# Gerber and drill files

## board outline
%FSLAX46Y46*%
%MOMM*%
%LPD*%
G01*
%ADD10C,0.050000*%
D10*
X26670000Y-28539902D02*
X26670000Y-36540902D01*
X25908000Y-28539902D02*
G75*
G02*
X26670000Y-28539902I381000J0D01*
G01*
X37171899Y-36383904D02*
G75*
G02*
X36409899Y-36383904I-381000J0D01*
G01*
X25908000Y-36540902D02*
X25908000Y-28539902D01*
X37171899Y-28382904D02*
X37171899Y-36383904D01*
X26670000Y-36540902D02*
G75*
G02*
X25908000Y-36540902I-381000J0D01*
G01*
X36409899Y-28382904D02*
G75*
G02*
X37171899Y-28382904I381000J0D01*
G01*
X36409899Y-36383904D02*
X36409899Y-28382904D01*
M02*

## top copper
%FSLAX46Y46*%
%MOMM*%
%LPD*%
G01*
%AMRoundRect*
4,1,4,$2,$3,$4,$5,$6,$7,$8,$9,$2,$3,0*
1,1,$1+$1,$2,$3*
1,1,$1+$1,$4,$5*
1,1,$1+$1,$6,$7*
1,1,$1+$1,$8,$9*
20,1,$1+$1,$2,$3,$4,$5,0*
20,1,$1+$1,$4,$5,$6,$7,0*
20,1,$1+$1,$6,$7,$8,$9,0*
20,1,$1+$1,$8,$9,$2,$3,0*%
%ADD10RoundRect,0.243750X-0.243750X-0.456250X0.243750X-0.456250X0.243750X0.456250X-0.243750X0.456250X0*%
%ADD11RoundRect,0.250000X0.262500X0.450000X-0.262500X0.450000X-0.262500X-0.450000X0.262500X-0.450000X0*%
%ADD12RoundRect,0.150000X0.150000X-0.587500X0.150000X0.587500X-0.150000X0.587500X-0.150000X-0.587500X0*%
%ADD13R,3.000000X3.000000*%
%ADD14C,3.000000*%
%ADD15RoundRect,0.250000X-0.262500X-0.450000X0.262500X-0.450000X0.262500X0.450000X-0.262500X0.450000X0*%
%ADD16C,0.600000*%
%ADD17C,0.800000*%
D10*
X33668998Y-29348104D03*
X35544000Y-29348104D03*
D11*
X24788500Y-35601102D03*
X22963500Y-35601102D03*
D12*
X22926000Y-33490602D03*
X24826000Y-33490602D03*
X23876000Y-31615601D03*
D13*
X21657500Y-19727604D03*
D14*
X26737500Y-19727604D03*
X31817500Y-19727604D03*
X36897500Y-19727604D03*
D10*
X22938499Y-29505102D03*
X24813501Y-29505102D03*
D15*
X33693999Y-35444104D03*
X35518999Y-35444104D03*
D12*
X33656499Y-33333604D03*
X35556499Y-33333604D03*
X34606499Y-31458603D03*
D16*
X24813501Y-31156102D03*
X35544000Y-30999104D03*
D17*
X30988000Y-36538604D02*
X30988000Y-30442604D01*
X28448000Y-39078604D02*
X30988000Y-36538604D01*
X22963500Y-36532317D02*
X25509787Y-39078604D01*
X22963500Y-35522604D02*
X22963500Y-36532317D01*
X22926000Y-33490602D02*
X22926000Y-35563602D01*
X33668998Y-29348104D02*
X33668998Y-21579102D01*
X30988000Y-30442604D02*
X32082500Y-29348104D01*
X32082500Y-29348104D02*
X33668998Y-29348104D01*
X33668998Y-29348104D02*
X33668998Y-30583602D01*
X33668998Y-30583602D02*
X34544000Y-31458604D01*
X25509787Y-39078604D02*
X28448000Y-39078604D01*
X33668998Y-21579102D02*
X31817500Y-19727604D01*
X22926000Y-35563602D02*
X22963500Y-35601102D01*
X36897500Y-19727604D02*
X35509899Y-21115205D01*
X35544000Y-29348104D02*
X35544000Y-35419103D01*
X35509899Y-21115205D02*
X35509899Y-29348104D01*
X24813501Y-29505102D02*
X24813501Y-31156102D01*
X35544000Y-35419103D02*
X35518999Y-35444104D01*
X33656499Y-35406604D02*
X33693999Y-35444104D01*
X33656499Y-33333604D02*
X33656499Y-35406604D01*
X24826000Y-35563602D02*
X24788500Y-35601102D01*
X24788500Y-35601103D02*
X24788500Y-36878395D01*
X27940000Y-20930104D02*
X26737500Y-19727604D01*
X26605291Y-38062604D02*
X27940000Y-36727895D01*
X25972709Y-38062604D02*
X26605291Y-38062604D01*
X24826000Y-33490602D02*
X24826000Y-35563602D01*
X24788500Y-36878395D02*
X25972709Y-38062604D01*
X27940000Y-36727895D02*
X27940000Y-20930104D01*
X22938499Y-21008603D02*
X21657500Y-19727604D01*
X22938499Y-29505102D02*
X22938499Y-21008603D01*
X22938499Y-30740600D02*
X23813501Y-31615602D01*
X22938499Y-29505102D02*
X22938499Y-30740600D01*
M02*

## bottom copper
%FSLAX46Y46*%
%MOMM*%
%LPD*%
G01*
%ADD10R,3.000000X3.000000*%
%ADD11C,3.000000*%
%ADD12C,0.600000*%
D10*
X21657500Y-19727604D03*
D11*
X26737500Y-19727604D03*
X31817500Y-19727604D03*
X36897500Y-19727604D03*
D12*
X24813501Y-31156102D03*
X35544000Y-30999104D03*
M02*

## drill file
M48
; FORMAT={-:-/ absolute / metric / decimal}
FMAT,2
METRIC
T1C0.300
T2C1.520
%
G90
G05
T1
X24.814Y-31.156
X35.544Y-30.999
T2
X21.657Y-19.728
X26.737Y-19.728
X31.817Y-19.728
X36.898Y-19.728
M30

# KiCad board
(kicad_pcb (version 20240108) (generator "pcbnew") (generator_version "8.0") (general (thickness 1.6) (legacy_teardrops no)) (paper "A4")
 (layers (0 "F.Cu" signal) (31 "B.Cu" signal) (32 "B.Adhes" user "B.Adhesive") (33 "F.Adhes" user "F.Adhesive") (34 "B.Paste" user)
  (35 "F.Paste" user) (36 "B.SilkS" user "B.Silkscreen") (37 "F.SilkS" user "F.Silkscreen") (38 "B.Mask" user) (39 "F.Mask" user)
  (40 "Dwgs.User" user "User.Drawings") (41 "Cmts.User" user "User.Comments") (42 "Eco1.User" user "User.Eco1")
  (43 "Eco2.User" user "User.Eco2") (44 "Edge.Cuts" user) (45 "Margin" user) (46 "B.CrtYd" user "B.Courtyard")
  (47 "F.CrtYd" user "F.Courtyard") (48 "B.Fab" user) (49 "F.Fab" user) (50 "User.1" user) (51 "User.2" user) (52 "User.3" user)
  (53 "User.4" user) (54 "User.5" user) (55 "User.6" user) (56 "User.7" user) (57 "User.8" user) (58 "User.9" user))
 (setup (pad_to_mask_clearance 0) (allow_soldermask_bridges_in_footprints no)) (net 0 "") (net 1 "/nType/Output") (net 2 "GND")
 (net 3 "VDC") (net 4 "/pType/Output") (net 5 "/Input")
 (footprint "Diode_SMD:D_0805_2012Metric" (layer "F.Cu") (at 34.606499 29.348104)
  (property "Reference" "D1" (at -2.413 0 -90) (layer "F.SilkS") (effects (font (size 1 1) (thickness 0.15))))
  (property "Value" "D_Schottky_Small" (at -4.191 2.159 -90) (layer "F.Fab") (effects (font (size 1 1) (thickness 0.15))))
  (pad "1" smd roundrect (at -0.937501 0) (size 0.975 1.4) (layers "F.Cu" "F.Paste" "F.Mask") (roundrect_rratio 0.25)
   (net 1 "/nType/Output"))
  (pad "2" smd roundrect (at 0.937501 0) (size 0.975 1.4) (layers "F.Cu" "F.Paste" "F.Mask") (roundrect_rratio 0.25) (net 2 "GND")))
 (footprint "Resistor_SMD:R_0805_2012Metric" (layer "F.Cu") (at 23.876 35.601102 180)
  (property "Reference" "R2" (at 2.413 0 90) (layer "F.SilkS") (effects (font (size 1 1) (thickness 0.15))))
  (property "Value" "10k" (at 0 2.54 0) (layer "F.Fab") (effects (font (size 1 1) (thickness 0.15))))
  (pad "1" smd roundrect (at -0.9125 0 180) (size 1.025 1.4) (layers "F.Cu" "F.Paste" "F.Mask") (roundrect_rratio 0.243902) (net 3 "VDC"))
  (pad "2" smd roundrect (at 0.9125 0 180) (size 1.025 1.4) (layers "F.Cu" "F.Paste" "F.Mask") (roundrect_rratio 0.243902)
   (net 1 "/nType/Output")))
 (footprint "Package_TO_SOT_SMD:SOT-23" (layer "F.Cu") (at 23.876 32.553102 90)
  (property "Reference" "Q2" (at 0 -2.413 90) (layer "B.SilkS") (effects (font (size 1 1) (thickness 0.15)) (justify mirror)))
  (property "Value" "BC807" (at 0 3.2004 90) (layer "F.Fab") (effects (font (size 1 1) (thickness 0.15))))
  (pad "1" smd roundrect (at -0.9375 -0.95 90) (size 1.475 0.6) (layers "F.Cu" "F.Paste" "F.Mask") (roundrect_rratio 0.25)
   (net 1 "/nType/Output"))
  (pad "2" smd roundrect (at -0.9375 0.95 90) (size 1.475 0.6) (layers "F.Cu" "F.Paste" "F.Mask") (roundrect_rratio 0.25) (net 3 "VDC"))
  (pad "3" smd roundrect (at 0.937501 0 90) (size 1.475 0.6) (layers "F.Cu" "F.Paste" "F.Mask") (roundrect_rratio 0.25)
   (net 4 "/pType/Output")))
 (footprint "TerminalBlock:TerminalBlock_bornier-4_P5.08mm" (layer "F.Cu") (at 21.6575 19.727604)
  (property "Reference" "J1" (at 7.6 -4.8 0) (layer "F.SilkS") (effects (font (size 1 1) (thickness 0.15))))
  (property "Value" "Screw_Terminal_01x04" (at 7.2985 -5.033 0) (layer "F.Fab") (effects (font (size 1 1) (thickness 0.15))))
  (pad "1" thru_hole rect (at 0 0) (size 3 3) (drill 1.52) (layers "*.Cu" "*.Mask") (remove_unused_layers no) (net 4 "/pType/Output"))
  (pad "2" thru_hole circle (at 5.08 0) (size 3 3) (drill 1.52) (layers "*.Cu" "*.Mask") (remove_unused_layers no) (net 3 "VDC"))
  (pad "3" thru_hole circle (at 10.16 0) (size 3 3) (drill 1.52) (layers "*.Cu" "*.Mask") (remove_unused_layers no) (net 1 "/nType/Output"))
  (pad "4" thru_hole circle (at 15.24 0) (size 3 3) (drill 1.52) (layers "*.Cu" "*.Mask") (remove_unused_layers no) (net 2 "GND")))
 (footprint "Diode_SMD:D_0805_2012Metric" (layer "F.Cu") (at 23.876 29.505102)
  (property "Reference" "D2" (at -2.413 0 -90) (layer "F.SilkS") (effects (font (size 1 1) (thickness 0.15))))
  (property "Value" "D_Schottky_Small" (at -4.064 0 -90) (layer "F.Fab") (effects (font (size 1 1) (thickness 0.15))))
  (pad "1" smd roundrect (at -0.937501 0) (size 0.975 1.4) (layers "F.Cu" "F.Paste" "F.Mask") (roundrect_rratio 0.25)
   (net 4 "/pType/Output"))
  (pad "2" smd roundrect (at 0.937501 0) (size 0.975 1.4) (layers "F.Cu" "F.Paste" "F.Mask") (roundrect_rratio 0.25) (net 2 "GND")))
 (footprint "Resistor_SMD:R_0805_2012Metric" (layer "F.Cu") (at 34.606499 35.444104)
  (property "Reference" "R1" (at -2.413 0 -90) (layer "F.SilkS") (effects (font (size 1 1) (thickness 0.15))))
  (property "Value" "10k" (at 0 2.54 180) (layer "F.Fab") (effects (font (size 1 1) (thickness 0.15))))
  (pad "1" smd roundrect (at -0.9125 0) (size 1.025 1.4) (layers "F.Cu" "F.Paste" "F.Mask") (roundrect_rratio 0.243902) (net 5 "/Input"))
  (pad "2" smd roundrect (at 0.9125 0) (size 1.025 1.4) (layers "F.Cu" "F.Paste" "F.Mask") (roundrect_rratio 0.243902) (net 2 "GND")))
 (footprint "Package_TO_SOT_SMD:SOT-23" (layer "F.Cu") (at 34.606499 32.396104 90)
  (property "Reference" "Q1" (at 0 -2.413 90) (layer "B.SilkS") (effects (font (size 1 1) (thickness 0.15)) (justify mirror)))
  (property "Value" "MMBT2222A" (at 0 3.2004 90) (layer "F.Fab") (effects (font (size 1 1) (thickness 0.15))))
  (pad "1" smd roundrect (at -0.9375 -0.95 90) (size 1.475 0.6) (layers "F.Cu" "F.Paste" "F.Mask") (roundrect_rratio 0.25) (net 5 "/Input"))
  (pad "2" smd roundrect (at -0.9375 0.95 90) (size 1.475 0.6) (layers "F.Cu" "F.Paste" "F.Mask") (roundrect_rratio 0.25) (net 2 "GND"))
  (pad "3" smd roundrect (at 0.937501 0 90) (size 1.475 0.6) (layers "F.Cu" "F.Paste" "F.Mask") (roundrect_rratio 0.25)
   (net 1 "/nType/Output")))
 (gr_line (start 26.67 28.539902) (end 26.67 36.540902) (stroke (width 0.05) (type default)) (layer "Edge.Cuts"))
 (gr_arc (start 25.908 28.539902) (mid 26.289 28.158902) (end 26.67 28.539902) (stroke (width 0.05) (type default)) (layer "Edge.Cuts"))
 (gr_arc (start 37.171899 36.383904) (mid 36.790899 36.764904) (end 36.409899 36.383904) (stroke (width 0.05) (type default))
  (layer "Edge.Cuts"))
 (gr_line (start 25.908 36.540902) (end 25.908 28.539902) (stroke (width 0.05) (type default)) (layer "Edge.Cuts"))
 (gr_line (start 37.171899 28.382904) (end 37.171899 36.383904) (stroke (width 0.05) (type default)) (layer "Edge.Cuts"))
 (gr_arc (start 26.67 36.540902) (mid 26.289 36.921902) (end 25.908 36.540902) (stroke (width 0.05) (type default)) (layer "Edge.Cuts"))
 (gr_arc (start 36.409899 28.382904) (mid 36.790899 28.001904) (end 37.171899 28.382904) (stroke (width 0.05) (type default))
  (layer "Edge.Cuts"))
 (gr_line (start 36.409899 36.383904) (end 36.409899 28.382904) (stroke (width 0.05) (type default)) (layer "Edge.Cuts"))
 (segment (start 30.988 36.538604) (end 30.988 30.442604) (width 0.8) (layer "F.Cu") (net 1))
 (segment (start 28.448 39.078604) (end 30.988 36.538604) (width 0.8) (layer "F.Cu") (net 1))
 (segment (start 22.9635 36.532317) (end 25.509787 39.078604) (width 0.8) (layer "F.Cu") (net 1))
 (segment (start 22.9635 35.522604) (end 22.9635 36.532317) (width 0.8) (layer "F.Cu") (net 1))
 (segment (start 22.926 33.490602) (end 22.926 35.563602) (width 0.8) (layer "F.Cu") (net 1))
 (segment (start 33.668998 29.348104) (end 33.668998 21.579102) (width 0.8) (layer "F.Cu") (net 1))
 (segment (start 30.988 30.442604) (end 32.0825 29.348104) (width 0.8) (layer "F.Cu") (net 1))
 (segment (start 32.0825 29.348104) (end 33.668998 29.348104) (width 0.8) (layer "F.Cu") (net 1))
 (segment (start 33.668998 29.348104) (end 33.668998 30.583602) (width 0.8) (layer "F.Cu") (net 1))
 (segment (start 33.668998 30.583602) (end 34.544 31.458604) (width 0.8) (layer "F.Cu") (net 1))
 (segment (start 25.509787 39.078604) (end 28.448 39.078604) (width 0.8) (layer "F.Cu") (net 1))
 (segment (start 33.668998 21.579102) (end 31.8175 19.727604) (width 0.8) (layer "F.Cu") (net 1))
 (segment (start 22.926 35.563602) (end 22.9635 35.601102) (width 0.8) (layer "F.Cu") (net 1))
 (segment (start 36.8975 19.727604) (end 35.509899 21.115205) (width 0.8) (layer "F.Cu") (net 2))
 (segment (start 35.544 29.348104) (end 35.544 35.419103) (width 0.8) (layer "F.Cu") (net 2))
 (segment (start 35.509899 21.115205) (end 35.509899 29.348104) (width 0.8) (layer "F.Cu") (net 2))
 (segment (start 24.813501 29.505102) (end 24.813501 31.156102) (width 0.8) (layer "F.Cu") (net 2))
 (segment (start 35.544 35.419103) (end 35.518999 35.444104) (width 0.8) (layer "F.Cu") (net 2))
 (via (at 24.813501 31.156102) (size 0.6) (drill 0.3) (layers "F.Cu" "B.Cu") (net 2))
 (via (at 35.544 30.999104) (size 0.6) (drill 0.3) (layers "F.Cu" "B.Cu") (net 2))
 (segment (start 33.656499 35.406604) (end 33.693999 35.444104) (width 0.8) (layer "F.Cu") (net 5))
 (segment (start 33.656499 33.333604) (end 33.656499 35.406604) (width 0.8) (layer "F.Cu") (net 5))
 (segment (start 24.826 35.563602) (end 24.7885 35.601102) (width 0.8) (layer "F.Cu") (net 3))
 (segment (start 24.7885 35.601103) (end 24.7885 36.878395) (width 0.8) (layer "F.Cu") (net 3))
 (segment (start 27.94 20.930104) (end 26.7375 19.727604) (width 0.8) (layer "F.Cu") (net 3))
 (segment (start 26.605291 38.062604) (end 27.94 36.727895) (width 0.8) (layer "F.Cu") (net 3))
 (segment (start 25.972709 38.062604) (end 26.605291 38.062604) (width 0.8) (layer "F.Cu") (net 3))
 (segment (start 24.826 33.490602) (end 24.826 35.563602) (width 0.8) (layer "F.Cu") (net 3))
 (segment (start 24.7885 36.878395) (end 25.972709 38.062604) (width 0.8) (layer "F.Cu") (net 3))
 (segment (start 27.94 36.727895) (end 27.94 20.930104) (width 0.8) (layer "F.Cu") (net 3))
 (segment (start 22.938499 21.008603) (end 21.6575 19.727604) (width 0.8) (layer "F.Cu") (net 4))
 (segment (start 22.938499 29.505102) (end 22.938499 21.008603) (width 0.8) (layer "F.Cu") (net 4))
 (segment (start 22.938499 30.7406) (end 23.813501 31.615602) (width 0.8) (layer "F.Cu") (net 4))
 (segment (start 22.938499 29.505102) (end 22.938499 30.7406) (width 0.8) (layer "F.Cu") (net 4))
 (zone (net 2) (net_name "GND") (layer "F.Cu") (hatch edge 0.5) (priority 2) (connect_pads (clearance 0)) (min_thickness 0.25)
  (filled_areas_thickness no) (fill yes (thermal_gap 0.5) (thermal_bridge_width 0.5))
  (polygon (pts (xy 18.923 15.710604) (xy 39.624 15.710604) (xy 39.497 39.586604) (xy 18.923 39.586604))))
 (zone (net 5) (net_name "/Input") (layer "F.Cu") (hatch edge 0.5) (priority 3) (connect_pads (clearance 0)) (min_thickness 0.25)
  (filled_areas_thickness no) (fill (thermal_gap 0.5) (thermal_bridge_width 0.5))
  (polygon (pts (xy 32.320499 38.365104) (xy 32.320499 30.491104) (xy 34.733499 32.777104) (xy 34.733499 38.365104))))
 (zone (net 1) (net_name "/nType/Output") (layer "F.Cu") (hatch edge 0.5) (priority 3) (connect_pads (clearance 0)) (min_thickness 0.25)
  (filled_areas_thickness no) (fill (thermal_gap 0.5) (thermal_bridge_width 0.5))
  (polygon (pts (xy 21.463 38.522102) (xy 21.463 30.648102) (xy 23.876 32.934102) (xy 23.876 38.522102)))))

